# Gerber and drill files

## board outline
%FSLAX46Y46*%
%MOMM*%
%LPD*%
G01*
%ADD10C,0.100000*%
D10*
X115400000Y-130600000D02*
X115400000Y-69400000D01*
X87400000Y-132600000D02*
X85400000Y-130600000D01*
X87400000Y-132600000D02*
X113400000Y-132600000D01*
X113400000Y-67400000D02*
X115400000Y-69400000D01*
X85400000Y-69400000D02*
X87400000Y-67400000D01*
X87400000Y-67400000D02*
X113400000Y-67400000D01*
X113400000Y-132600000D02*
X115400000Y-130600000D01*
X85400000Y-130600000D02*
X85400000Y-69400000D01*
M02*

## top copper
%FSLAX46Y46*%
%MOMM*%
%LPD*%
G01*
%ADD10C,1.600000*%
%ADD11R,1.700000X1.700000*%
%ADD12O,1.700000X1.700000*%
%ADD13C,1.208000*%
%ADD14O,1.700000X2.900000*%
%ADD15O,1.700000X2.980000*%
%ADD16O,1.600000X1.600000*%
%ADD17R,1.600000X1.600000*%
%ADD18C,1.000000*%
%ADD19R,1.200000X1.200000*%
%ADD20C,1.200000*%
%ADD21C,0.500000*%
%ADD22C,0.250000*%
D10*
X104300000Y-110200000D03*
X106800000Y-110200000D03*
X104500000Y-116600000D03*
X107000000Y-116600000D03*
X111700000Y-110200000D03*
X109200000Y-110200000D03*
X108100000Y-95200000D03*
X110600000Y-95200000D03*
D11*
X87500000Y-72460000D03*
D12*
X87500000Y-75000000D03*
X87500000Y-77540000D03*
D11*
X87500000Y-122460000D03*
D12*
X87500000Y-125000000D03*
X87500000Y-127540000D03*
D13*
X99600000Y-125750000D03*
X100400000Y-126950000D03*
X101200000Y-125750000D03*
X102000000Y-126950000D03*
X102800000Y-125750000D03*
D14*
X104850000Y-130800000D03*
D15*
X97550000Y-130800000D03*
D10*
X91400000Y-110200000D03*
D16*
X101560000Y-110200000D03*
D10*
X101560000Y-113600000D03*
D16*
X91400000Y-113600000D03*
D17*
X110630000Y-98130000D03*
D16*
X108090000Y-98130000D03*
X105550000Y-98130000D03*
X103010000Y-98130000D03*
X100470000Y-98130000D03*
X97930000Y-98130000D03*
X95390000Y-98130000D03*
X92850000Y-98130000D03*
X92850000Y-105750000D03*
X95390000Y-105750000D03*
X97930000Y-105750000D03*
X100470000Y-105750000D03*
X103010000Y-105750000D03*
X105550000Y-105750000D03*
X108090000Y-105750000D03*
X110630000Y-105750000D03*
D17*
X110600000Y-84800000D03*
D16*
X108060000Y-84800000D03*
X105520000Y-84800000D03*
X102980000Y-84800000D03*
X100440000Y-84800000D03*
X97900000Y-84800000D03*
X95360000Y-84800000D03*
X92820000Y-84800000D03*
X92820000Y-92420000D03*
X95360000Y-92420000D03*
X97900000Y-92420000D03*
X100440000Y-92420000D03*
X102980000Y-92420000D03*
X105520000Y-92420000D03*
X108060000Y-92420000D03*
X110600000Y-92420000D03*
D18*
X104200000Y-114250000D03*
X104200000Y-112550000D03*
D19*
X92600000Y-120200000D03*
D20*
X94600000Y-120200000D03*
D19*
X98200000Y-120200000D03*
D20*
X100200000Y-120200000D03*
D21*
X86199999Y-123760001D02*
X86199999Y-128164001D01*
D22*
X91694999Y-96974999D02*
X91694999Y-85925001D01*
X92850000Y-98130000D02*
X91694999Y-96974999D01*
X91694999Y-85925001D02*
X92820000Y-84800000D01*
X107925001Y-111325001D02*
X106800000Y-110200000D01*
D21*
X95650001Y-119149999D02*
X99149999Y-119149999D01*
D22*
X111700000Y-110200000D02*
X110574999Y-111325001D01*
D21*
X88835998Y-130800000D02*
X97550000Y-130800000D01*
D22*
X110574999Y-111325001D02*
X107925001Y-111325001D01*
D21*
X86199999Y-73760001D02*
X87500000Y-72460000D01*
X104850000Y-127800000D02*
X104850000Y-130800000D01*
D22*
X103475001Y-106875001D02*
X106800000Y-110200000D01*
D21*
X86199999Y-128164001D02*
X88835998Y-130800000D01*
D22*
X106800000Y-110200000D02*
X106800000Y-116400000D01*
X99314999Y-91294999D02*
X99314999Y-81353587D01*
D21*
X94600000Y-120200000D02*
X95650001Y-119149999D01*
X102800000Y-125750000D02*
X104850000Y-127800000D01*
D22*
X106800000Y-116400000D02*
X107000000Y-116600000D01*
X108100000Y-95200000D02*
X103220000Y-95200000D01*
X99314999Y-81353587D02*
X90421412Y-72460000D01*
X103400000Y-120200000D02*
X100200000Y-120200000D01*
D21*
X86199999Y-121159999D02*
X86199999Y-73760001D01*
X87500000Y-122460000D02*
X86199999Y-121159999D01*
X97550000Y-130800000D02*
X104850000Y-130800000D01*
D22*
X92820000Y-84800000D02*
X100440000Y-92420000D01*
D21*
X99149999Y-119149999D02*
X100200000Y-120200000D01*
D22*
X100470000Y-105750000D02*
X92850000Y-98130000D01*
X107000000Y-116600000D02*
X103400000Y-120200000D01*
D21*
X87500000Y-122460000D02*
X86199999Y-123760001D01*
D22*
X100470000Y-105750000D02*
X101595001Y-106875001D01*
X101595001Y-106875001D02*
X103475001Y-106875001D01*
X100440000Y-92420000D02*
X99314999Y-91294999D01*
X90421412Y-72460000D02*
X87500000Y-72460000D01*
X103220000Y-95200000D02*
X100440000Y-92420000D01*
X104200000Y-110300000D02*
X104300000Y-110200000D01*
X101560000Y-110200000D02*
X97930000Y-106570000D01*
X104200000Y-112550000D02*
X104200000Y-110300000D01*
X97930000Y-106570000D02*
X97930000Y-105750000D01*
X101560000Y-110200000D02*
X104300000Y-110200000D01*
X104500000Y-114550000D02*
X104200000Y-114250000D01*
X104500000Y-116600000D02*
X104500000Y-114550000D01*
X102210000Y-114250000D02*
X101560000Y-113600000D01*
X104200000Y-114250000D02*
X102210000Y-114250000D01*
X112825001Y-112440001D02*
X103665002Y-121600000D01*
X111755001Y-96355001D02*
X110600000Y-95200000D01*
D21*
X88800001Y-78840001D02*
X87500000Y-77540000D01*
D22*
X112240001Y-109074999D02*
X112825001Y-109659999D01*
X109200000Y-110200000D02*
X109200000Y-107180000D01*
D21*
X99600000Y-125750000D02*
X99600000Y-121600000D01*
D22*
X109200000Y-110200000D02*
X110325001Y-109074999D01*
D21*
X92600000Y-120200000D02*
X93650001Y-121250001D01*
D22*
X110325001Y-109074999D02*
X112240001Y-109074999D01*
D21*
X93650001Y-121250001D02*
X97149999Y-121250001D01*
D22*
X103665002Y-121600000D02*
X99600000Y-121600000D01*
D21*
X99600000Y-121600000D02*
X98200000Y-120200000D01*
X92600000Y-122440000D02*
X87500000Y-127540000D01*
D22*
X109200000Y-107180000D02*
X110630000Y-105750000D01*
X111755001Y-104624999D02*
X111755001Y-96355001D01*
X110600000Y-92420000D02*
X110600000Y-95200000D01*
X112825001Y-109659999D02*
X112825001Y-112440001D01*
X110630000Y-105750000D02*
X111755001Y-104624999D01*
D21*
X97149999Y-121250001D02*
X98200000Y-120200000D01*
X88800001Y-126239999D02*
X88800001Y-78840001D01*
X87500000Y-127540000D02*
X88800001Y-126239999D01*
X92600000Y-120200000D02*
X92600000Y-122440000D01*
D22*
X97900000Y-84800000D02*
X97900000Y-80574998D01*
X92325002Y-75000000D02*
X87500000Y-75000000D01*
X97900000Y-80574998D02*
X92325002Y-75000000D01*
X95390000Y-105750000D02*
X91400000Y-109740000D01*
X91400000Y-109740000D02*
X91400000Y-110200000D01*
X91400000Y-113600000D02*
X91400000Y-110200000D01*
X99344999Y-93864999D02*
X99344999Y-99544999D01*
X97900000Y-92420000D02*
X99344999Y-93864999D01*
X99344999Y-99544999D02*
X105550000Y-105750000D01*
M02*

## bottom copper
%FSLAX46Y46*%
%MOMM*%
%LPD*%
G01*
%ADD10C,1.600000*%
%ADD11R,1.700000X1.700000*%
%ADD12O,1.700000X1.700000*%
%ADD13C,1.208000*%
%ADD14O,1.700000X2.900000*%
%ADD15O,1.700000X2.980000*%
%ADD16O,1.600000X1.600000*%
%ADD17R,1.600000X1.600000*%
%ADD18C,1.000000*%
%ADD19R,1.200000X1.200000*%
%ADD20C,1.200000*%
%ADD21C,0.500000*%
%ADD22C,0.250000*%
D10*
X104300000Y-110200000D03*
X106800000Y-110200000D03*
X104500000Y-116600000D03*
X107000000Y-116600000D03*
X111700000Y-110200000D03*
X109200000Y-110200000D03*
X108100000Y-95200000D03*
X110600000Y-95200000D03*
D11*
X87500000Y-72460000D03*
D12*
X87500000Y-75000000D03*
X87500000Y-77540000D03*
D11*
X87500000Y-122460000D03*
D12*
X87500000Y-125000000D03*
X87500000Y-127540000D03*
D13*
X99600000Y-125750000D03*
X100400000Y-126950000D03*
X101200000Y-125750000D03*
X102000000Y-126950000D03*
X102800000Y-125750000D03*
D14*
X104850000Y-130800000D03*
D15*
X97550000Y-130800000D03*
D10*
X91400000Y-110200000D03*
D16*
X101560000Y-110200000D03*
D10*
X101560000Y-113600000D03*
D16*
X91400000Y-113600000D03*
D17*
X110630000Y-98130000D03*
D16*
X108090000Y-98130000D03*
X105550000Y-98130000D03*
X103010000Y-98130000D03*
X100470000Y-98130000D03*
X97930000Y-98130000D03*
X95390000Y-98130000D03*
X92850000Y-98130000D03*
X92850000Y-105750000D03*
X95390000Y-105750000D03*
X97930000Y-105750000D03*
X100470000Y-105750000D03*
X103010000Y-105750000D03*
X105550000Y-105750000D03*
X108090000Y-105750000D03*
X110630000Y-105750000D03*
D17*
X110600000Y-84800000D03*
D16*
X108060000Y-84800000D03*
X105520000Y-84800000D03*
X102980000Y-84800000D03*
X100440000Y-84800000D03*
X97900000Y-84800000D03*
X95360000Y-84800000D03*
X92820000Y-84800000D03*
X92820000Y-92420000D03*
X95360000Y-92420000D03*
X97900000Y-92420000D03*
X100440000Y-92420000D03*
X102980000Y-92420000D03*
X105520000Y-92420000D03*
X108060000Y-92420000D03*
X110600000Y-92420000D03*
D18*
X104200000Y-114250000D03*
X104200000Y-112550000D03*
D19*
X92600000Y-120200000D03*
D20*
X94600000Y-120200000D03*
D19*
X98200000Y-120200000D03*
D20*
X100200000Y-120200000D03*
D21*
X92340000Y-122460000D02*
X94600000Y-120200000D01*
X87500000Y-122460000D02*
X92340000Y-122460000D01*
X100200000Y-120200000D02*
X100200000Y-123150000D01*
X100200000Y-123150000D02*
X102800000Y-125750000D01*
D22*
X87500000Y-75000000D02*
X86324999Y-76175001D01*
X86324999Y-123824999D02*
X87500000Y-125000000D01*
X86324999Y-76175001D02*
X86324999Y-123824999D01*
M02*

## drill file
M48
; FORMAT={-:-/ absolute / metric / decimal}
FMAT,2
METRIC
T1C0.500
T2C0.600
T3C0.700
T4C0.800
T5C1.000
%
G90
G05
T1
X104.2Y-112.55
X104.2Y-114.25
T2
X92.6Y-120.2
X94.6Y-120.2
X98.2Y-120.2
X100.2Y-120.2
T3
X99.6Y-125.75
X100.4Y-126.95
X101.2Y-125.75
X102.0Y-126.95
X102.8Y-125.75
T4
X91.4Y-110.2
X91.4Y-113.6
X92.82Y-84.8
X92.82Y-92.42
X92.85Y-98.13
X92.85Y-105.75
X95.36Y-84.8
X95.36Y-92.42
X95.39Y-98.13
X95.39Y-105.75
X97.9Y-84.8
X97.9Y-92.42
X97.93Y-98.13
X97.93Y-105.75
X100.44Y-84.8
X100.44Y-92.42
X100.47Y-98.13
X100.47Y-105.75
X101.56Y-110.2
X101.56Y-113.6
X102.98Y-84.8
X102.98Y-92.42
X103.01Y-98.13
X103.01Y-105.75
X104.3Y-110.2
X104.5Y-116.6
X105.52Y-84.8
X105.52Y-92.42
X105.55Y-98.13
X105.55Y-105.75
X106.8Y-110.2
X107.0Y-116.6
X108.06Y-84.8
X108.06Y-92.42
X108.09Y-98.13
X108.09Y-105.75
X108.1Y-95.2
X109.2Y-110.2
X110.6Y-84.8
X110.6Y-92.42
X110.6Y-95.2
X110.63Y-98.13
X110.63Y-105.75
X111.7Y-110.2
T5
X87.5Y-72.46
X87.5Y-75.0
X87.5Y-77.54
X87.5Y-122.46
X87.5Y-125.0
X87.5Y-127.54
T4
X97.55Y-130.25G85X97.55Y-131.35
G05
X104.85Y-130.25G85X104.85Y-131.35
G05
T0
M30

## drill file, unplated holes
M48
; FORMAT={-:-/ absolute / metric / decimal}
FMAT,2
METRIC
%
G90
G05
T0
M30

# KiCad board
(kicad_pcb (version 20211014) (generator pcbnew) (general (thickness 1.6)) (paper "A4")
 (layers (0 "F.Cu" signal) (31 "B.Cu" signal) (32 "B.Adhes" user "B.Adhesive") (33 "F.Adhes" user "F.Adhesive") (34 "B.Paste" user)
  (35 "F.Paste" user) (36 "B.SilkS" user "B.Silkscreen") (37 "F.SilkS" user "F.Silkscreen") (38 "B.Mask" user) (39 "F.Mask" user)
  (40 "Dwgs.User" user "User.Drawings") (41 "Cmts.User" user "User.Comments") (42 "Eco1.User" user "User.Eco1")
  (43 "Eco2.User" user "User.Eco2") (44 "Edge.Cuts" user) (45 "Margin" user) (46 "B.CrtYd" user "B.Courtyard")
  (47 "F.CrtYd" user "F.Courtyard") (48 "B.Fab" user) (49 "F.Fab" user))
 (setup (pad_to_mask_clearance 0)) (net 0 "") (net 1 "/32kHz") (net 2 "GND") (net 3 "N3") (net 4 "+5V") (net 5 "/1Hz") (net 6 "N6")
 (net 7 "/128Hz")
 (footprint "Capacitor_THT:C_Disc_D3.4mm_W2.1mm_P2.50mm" (layer "F.Cu") (at 104.3 110.2)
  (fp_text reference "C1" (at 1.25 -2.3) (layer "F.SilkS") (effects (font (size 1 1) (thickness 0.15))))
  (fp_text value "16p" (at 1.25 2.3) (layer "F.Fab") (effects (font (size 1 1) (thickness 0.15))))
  (pad "1" thru_hole circle locked (at 0 0) (size 1.6 1.6) (drill 0.8) (layers *.Cu *.Mask) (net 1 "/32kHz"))
  (pad "2" thru_hole circle locked (at 2.5 0) (size 1.6 1.6) (drill 0.8) (layers *.Cu *.Mask) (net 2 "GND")))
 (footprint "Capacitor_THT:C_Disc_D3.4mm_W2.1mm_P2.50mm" (layer "F.Cu") (at 104.5 116.6)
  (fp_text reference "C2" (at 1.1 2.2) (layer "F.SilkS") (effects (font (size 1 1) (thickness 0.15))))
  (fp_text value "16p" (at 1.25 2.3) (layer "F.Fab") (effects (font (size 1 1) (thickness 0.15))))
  (pad "1" thru_hole circle locked (at 0 0) (size 1.6 1.6) (drill 0.8) (layers *.Cu *.Mask) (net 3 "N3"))
  (pad "2" thru_hole circle locked (at 2.5 0) (size 1.6 1.6) (drill 0.8) (layers *.Cu *.Mask) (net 2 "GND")))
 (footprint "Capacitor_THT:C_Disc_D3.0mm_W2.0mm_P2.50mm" (layer "F.Cu") (at 111.7 110.2 180)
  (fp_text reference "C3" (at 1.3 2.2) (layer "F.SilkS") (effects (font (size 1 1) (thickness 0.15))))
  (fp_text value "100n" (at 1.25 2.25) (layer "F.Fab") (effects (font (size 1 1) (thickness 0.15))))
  (pad "1" thru_hole circle locked (at 0 0 180) (size 1.6 1.6) (drill 0.8) (layers *.Cu *.Mask) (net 2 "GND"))
  (pad "2" thru_hole circle locked (at 2.5 0 180) (size 1.6 1.6) (drill 0.8) (layers *.Cu *.Mask) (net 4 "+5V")))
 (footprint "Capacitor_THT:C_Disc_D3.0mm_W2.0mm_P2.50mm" (layer "F.Cu") (at 108.1 95.2)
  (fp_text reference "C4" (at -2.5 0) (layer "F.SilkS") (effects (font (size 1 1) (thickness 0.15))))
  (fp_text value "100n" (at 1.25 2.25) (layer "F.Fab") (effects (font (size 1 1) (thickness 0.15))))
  (pad "1" thru_hole circle locked (at 0 0) (size 1.6 1.6) (drill 0.8) (layers *.Cu *.Mask) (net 2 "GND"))
  (pad "2" thru_hole circle locked (at 2.5 0) (size 1.6 1.6) (drill 0.8) (layers *.Cu *.Mask) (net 4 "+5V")))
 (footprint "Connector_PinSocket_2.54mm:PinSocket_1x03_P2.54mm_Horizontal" (layer "F.Cu") (at 87.5 72.46)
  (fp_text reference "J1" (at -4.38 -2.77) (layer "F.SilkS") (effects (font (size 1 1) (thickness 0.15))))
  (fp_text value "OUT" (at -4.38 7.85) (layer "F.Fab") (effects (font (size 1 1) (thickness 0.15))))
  (pad "1" thru_hole rect locked (at 0 0) (size 1.7 1.7) (drill 1) (layers *.Cu *.Mask) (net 2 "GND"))
  (pad "2" thru_hole oval locked (at 0 2.54) (size 1.7 1.7) (drill 1) (layers *.Cu *.Mask) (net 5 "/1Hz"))
  (pad "3" thru_hole oval locked (at 0 5.08) (size 1.7 1.7) (drill 1) (layers *.Cu *.Mask) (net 4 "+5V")))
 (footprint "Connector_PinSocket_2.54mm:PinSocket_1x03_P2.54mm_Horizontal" (layer "F.Cu") (at 87.5 122.46)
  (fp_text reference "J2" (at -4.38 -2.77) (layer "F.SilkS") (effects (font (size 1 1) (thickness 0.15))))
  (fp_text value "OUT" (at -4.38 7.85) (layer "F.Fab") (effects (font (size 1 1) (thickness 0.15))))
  (pad "1" thru_hole rect locked (at 0 0) (size 1.7 1.7) (drill 1) (layers *.Cu *.Mask) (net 2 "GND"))
  (pad "2" thru_hole oval locked (at 0 2.54) (size 1.7 1.7) (drill 1) (layers *.Cu *.Mask) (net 5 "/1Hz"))
  (pad "3" thru_hole oval locked (at 0 5.08) (size 1.7 1.7) (drill 1) (layers *.Cu *.Mask) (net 4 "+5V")))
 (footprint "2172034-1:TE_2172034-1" (layer "F.Cu") (at 101.2 130.8 -90)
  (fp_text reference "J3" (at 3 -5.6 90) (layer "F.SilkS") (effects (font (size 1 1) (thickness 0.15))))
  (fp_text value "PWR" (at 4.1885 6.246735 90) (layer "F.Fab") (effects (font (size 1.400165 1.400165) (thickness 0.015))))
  (pad "1" thru_hole circle locked (at -5.05 1.6 270) (size 1.208 1.208) (drill 0.7) (layers *.Cu *.Mask) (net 4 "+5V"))
  (pad "2" thru_hole circle locked (at -3.85 0.8 270) (size 1.208 1.208) (drill 0.7) (layers *.Cu *.Mask))
  (pad "3" thru_hole circle locked (at -5.05 0 270) (size 1.208 1.208) (drill 0.7) (layers *.Cu *.Mask))
  (pad "4" thru_hole circle locked (at -3.85 -0.8 270) (size 1.208 1.208) (drill 0.7) (layers *.Cu *.Mask))
  (pad "5" thru_hole circle locked (at -5.05 -1.6 270) (size 1.208 1.208) (drill 0.7) (layers *.Cu *.Mask) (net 2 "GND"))
  (pad "6" thru_hole oval locked (at 0 -3.65 270) (size 2.9 1.7) (drill oval 1.9 0.8) (layers *.Cu *.Mask) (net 2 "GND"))
  (pad "6" thru_hole oval locked (at 0 3.65 270) (size 2.98 1.7) (drill oval 1.9 0.8) (layers *.Cu *.Mask) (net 2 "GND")))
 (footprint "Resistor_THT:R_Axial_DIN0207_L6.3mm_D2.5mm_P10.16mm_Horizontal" (layer "F.Cu") (at 91.4 110.2)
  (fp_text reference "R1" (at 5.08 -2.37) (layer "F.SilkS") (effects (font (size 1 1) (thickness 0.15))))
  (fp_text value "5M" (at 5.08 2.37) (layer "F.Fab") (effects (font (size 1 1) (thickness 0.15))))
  (pad "1" thru_hole circle locked (at 0 0) (size 1.6 1.6) (drill 0.8) (layers *.Cu *.Mask) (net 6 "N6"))
  (pad "2" thru_hole oval locked (at 10.16 0) (size 1.6 1.6) (drill 0.8) (layers *.Cu *.Mask) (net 1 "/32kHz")))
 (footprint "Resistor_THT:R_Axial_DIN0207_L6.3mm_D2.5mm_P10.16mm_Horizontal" (layer "F.Cu") (at 101.56 113.6 180)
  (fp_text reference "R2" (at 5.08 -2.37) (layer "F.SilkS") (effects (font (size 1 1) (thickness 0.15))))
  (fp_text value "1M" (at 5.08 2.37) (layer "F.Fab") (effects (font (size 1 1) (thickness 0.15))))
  (pad "1" thru_hole circle locked (at 0 0 180) (size 1.6 1.6) (drill 0.8) (layers *.Cu *.Mask) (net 3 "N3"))
  (pad "2" thru_hole oval locked (at 10.16 0 180) (size 1.6 1.6) (drill 0.8) (layers *.Cu *.Mask) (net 6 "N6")))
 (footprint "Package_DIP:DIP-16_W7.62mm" (layer "F.Cu") (at 110.63 98.13 -90)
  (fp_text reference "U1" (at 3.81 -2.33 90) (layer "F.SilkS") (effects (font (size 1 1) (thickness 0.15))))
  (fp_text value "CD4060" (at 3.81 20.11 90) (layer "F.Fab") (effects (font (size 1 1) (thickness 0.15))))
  (pad "1" thru_hole rect locked (at 0 0 270) (size 1.6 1.6) (drill 0.8) (layers *.Cu *.Mask))
  (pad "2" thru_hole oval locked (at 0 2.54 270) (size 1.6 1.6) (drill 0.8) (layers *.Cu *.Mask))
  (pad "3" thru_hole oval locked (at 0 5.08 270) (size 1.6 1.6) (drill 0.8) (layers *.Cu *.Mask))
  (pad "4" thru_hole oval locked (at 0 7.62 270) (size 1.6 1.6) (drill 0.8) (layers *.Cu *.Mask))
  (pad "5" thru_hole oval locked (at 0 10.16 270) (size 1.6 1.6) (drill 0.8) (layers *.Cu *.Mask))
  (pad "6" thru_hole oval locked (at 0 12.7 270) (size 1.6 1.6) (drill 0.8) (layers *.Cu *.Mask))
  (pad "7" thru_hole oval locked (at 0 15.24 270) (size 1.6 1.6) (drill 0.8) (layers *.Cu *.Mask))
  (pad "8" thru_hole oval locked (at 0 17.78 270) (size 1.6 1.6) (drill 0.8) (layers *.Cu *.Mask) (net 2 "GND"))
  (pad "9" thru_hole oval locked (at 7.62 17.78 270) (size 1.6 1.6) (drill 0.8) (layers *.Cu *.Mask))
  (pad "10" thru_hole oval locked (at 7.62 15.24 270) (size 1.6 1.6) (drill 0.8) (layers *.Cu *.Mask) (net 6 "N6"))
  (pad "11" thru_hole oval locked (at 7.62 12.7 270) (size 1.6 1.6) (drill 0.8) (layers *.Cu *.Mask) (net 1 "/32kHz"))
  (pad "12" thru_hole oval locked (at 7.62 10.16 270) (size 1.6 1.6) (drill 0.8) (layers *.Cu *.Mask) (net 2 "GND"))
  (pad "13" thru_hole oval locked (at 7.62 7.62 270) (size 1.6 1.6) (drill 0.8) (layers *.Cu *.Mask))
  (pad "14" thru_hole oval locked (at 7.62 5.08 270) (size 1.6 1.6) (drill 0.8) (layers *.Cu *.Mask) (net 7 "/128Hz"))
  (pad "15" thru_hole oval locked (at 7.62 2.54 270) (size 1.6 1.6) (drill 0.8) (layers *.Cu *.Mask))
  (pad "16" thru_hole oval locked (at 7.62 0 270) (size 1.6 1.6) (drill 0.8) (layers *.Cu *.Mask) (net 4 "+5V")))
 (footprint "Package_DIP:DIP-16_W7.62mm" (layer "F.Cu") (at 110.6 84.8 -90)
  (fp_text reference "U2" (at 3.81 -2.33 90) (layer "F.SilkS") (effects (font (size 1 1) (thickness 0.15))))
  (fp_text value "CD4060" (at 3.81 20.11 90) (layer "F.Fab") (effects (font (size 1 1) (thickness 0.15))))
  (pad "1" thru_hole rect locked (at 0 0 270) (size 1.6 1.6) (drill 0.8) (layers *.Cu *.Mask))
  (pad "2" thru_hole oval locked (at 0 2.54 270) (size 1.6 1.6) (drill 0.8) (layers *.Cu *.Mask))
  (pad "3" thru_hole oval locked (at 0 5.08 270) (size 1.6 1.6) (drill 0.8) (layers *.Cu *.Mask))
  (pad "4" thru_hole oval locked (at 0 7.62 270) (size 1.6 1.6) (drill 0.8) (layers *.Cu *.Mask))
  (pad "5" thru_hole oval locked (at 0 10.16 270) (size 1.6 1.6) (drill 0.8) (layers *.Cu *.Mask))
  (pad "6" thru_hole oval locked (at 0 12.7 270) (size 1.6 1.6) (drill 0.8) (layers *.Cu *.Mask) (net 5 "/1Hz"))
  (pad "7" thru_hole oval locked (at 0 15.24 270) (size 1.6 1.6) (drill 0.8) (layers *.Cu *.Mask))
  (pad "8" thru_hole oval locked (at 0 17.78 270) (size 1.6 1.6) (drill 0.8) (layers *.Cu *.Mask) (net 2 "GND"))
  (pad "9" thru_hole oval locked (at 7.62 17.78 270) (size 1.6 1.6) (drill 0.8) (layers *.Cu *.Mask))
  (pad "10" thru_hole oval locked (at 7.62 15.24 270) (size 1.6 1.6) (drill 0.8) (layers *.Cu *.Mask))
  (pad "11" thru_hole oval locked (at 7.62 12.7 270) (size 1.6 1.6) (drill 0.8) (layers *.Cu *.Mask) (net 7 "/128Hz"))
  (pad "12" thru_hole oval locked (at 7.62 10.16 270) (size 1.6 1.6) (drill 0.8) (layers *.Cu *.Mask) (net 2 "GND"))
  (pad "13" thru_hole oval locked (at 7.62 7.62 270) (size 1.6 1.6) (drill 0.8) (layers *.Cu *.Mask))
  (pad "14" thru_hole oval locked (at 7.62 5.08 270) (size 1.6 1.6) (drill 0.8) (layers *.Cu *.Mask))
  (pad "15" thru_hole oval locked (at 7.62 2.54 270) (size 1.6 1.6) (drill 0.8) (layers *.Cu *.Mask))
  (pad "16" thru_hole oval locked (at 7.62 0 270) (size 1.6 1.6) (drill 0.8) (layers *.Cu *.Mask) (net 4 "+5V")))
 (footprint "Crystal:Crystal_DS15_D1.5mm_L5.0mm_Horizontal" (layer "F.Cu") (at 104.2 114.25 90)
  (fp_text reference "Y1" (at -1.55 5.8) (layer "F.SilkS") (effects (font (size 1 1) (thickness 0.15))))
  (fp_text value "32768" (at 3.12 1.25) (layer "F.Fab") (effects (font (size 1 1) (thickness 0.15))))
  (pad "1" thru_hole circle locked (at 0 0 90) (size 1 1) (drill 0.5) (layers *.Cu *.Mask) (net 3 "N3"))
  (pad "2" thru_hole circle locked (at 1.7 0 90) (size 1 1) (drill 0.5) (layers *.Cu *.Mask) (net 1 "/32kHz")))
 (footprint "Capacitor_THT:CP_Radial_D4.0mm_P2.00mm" (layer "F.Cu") (at 92.6 120.2)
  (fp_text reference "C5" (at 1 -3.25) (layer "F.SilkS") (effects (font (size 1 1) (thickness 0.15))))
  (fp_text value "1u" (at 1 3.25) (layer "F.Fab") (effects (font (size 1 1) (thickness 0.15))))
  (pad "1" thru_hole rect locked (at 0 0) (size 1.2 1.2) (drill 0.6) (layers *.Cu *.Mask) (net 4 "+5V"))
  (pad "2" thru_hole circle locked (at 2 0) (size 1.2 1.2) (drill 0.6) (layers *.Cu *.Mask) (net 2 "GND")))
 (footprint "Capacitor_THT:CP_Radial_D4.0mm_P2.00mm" (layer "F.Cu") (at 98.2 120.2)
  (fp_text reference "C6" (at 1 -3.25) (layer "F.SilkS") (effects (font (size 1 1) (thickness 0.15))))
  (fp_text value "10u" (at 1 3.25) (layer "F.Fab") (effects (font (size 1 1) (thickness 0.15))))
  (pad "1" thru_hole rect locked (at 0 0) (size 1.2 1.2) (drill 0.6) (layers *.Cu *.Mask) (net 4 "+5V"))
  (pad "2" thru_hole circle locked (at 2 0) (size 1.2 1.2) (drill 0.6) (layers *.Cu *.Mask) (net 2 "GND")))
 (gr_line (start 115.4 130.6) (end 115.4 69.4) (layer "Edge.Cuts") (width 0.1))
 (gr_line (start 87.4 132.6) (end 85.4 130.6) (layer "Edge.Cuts") (width 0.1))
 (gr_line (start 87.4 132.6) (end 113.4 132.6) (layer "Edge.Cuts") (width 0.1))
 (gr_line (start 113.4 67.4) (end 115.4 69.4) (layer "Edge.Cuts") (width 0.1))
 (gr_line (start 85.4 69.4) (end 87.4 67.4) (layer "Edge.Cuts") (width 0.1))
 (gr_line (start 87.4 67.4) (end 113.4 67.4) (layer "Edge.Cuts") (width 0.1))
 (gr_line (start 113.4 132.6) (end 115.4 130.6) (layer "Edge.Cuts") (width 0.1))
 (gr_line (start 85.4 130.6) (end 85.4 69.4) (layer "Edge.Cuts") (width 0.1))
 (segment (start 86.199999 123.760001) (end 86.199999 128.164001) (width 0.5) (layer "F.Cu") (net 2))
 (segment (start 91.694999 96.974999) (end 91.694999 85.925001) (width 0.25) (layer "F.Cu") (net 2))
 (segment (start 92.85 98.13) (end 91.694999 96.974999) (width 0.25) (layer "F.Cu") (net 2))
 (segment (start 91.694999 85.925001) (end 92.82 84.8) (width 0.25) (layer "F.Cu") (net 2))
 (segment (start 107.925001 111.325001) (end 106.8 110.2) (width 0.25) (layer "F.Cu") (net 2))
 (segment (start 95.650001 119.149999) (end 99.149999 119.149999) (width 0.5) (layer "F.Cu") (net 2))
 (segment (start 111.7 110.2) (end 110.574999 111.325001) (width 0.25) (layer "F.Cu") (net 2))
 (segment (start 88.835998 130.8) (end 97.55 130.8) (width 0.5) (layer "F.Cu") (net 2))
 (segment (start 110.574999 111.325001) (end 107.925001 111.325001) (width 0.25) (layer "F.Cu") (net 2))
 (segment (start 86.199999 73.760001) (end 87.5 72.46) (width 0.5) (layer "F.Cu") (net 2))
 (segment (start 104.85 127.8) (end 104.85 130.8) (width 0.5) (layer "F.Cu") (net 2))
 (segment (start 103.475001 106.875001) (end 106.8 110.2) (width 0.25) (layer "F.Cu") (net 2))
 (segment (start 86.199999 128.164001) (end 88.835998 130.8) (width 0.5) (layer "F.Cu") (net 2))
 (segment (start 106.8 110.2) (end 106.8 116.4) (width 0.25) (layer "F.Cu") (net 2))
 (segment (start 99.314999 91.294999) (end 99.314999 81.353587) (width 0.25) (layer "F.Cu") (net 2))
 (segment (start 94.6 120.2) (end 95.650001 119.149999) (width 0.5) (layer "F.Cu") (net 2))
 (segment (start 102.8 125.75) (end 104.85 127.8) (width 0.5) (layer "F.Cu") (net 2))
 (segment (start 106.8 116.4) (end 107 116.6) (width 0.25) (layer "F.Cu") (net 2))
 (segment (start 108.1 95.2) (end 103.22 95.2) (width 0.25) (layer "F.Cu") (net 2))
 (segment (start 99.314999 81.353587) (end 90.421412 72.46) (width 0.25) (layer "F.Cu") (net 2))
 (segment (start 103.4 120.2) (end 100.2 120.2) (width 0.25) (layer "F.Cu") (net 2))
 (segment (start 86.199999 121.159999) (end 86.199999 73.760001) (width 0.5) (layer "F.Cu") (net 2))
 (segment (start 87.5 122.46) (end 86.199999 121.159999) (width 0.5) (layer "F.Cu") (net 2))
 (segment (start 97.55 130.8) (end 104.85 130.8) (width 0.5) (layer "F.Cu") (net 2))
 (segment (start 92.82 84.8) (end 100.44 92.42) (width 0.25) (layer "F.Cu") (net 2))
 (segment (start 99.149999 119.149999) (end 100.2 120.2) (width 0.5) (layer "F.Cu") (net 2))
 (segment (start 100.47 105.75) (end 92.85 98.13) (width 0.25) (layer "F.Cu") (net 2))
 (segment (start 107 116.6) (end 103.4 120.2) (width 0.25) (layer "F.Cu") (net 2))
 (segment (start 87.5 122.46) (end 86.199999 123.760001) (width 0.5) (layer "F.Cu") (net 2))
 (segment (start 100.47 105.75) (end 101.595001 106.875001) (width 0.25) (layer "F.Cu") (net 2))
 (segment (start 101.595001 106.875001) (end 103.475001 106.875001) (width 0.25) (layer "F.Cu") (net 2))
 (segment (start 100.44 92.42) (end 99.314999 91.294999) (width 0.25) (layer "F.Cu") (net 2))
 (segment (start 90.421412 72.46) (end 87.5 72.46) (width 0.25) (layer "F.Cu") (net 2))
 (segment (start 103.22 95.2) (end 100.44 92.42) (width 0.25) (layer "F.Cu") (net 2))
 (segment (start 92.34 122.46) (end 94.6 120.2) (width 0.5) (layer "B.Cu") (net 2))
 (segment (start 87.5 122.46) (end 92.34 122.46) (width 0.5) (layer "B.Cu") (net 2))
 (segment (start 100.2 120.2) (end 100.2 123.15) (width 0.5) (layer "B.Cu") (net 2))
 (segment (start 100.2 123.15) (end 102.8 125.75) (width 0.5) (layer "B.Cu") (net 2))
 (segment (start 104.2 110.3) (end 104.3 110.2) (width 0.25) (layer "F.Cu") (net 1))
 (segment (start 101.56 110.2) (end 97.93 106.57) (width 0.25) (layer "F.Cu") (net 1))
 (segment (start 104.2 112.55) (end 104.2 110.3) (width 0.25) (layer "F.Cu") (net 1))
 (segment (start 97.93 106.57) (end 97.93 105.75) (width 0.25) (layer "F.Cu") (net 1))
 (segment (start 101.56 110.2) (end 104.3 110.2) (width 0.25) (layer "F.Cu") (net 1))
 (segment (start 104.5 114.55) (end 104.2 114.25) (width 0.25) (layer "F.Cu") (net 3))
 (segment (start 104.5 116.6) (end 104.5 114.55) (width 0.25) (layer "F.Cu") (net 3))
 (segment (start 102.21 114.25) (end 101.56 113.6) (width 0.25) (layer "F.Cu") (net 3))
 (segment (start 104.2 114.25) (end 102.21 114.25) (width 0.25) (layer "F.Cu") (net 3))
 (segment (start 112.825001 112.440001) (end 103.665002 121.6) (width 0.25) (layer "F.Cu") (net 4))
 (segment (start 111.755001 96.355001) (end 110.6 95.2) (width 0.25) (layer "F.Cu") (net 4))
 (segment (start 88.800001 78.840001) (end 87.5 77.54) (width 0.5) (layer "F.Cu") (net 4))
 (segment (start 112.240001 109.074999) (end 112.825001 109.659999) (width 0.25) (layer "F.Cu") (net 4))
 (segment (start 109.2 110.2) (end 109.2 107.18) (width 0.25) (layer "F.Cu") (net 4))
 (segment (start 99.6 125.75) (end 99.6 121.6) (width 0.5) (layer "F.Cu") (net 4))
 (segment (start 109.2 110.2) (end 110.325001 109.074999) (width 0.25) (layer "F.Cu") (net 4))
 (segment (start 92.6 120.2) (end 93.650001 121.250001) (width 0.5) (layer "F.Cu") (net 4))
 (segment (start 110.325001 109.074999) (end 112.240001 109.074999) (width 0.25) (layer "F.Cu") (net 4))
 (segment (start 93.650001 121.250001) (end 97.149999 121.250001) (width 0.5) (layer "F.Cu") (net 4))
 (segment (start 103.665002 121.6) (end 99.6 121.6) (width 0.25) (layer "F.Cu") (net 4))
 (segment (start 99.6 121.6) (end 98.2 120.2) (width 0.5) (layer "F.Cu") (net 4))
 (segment (start 92.6 122.44) (end 87.5 127.54) (width 0.5) (layer "F.Cu") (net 4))
 (segment (start 109.2 107.18) (end 110.63 105.75) (width 0.25) (layer "F.Cu") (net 4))
 (segment (start 111.755001 104.624999) (end 111.755001 96.355001) (width 0.25) (layer "F.Cu") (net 4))
 (segment (start 110.6 92.42) (end 110.6 95.2) (width 0.25) (layer "F.Cu") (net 4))
 (segment (start 112.825001 109.659999) (end 112.825001 112.440001) (width 0.25) (layer "F.Cu") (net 4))
 (segment (start 110.63 105.75) (end 111.755001 104.624999) (width 0.25) (layer "F.Cu") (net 4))
 (segment (start 97.149999 121.250001) (end 98.2 120.2) (width 0.5) (layer "F.Cu") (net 4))
 (segment (start 88.800001 126.239999) (end 88.800001 78.840001) (width 0.5) (layer "F.Cu") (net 4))
 (segment (start 87.5 127.54) (end 88.800001 126.239999) (width 0.5) (layer "F.Cu") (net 4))
 (segment (start 92.6 120.2) (end 92.6 122.44) (width 0.5) (layer "F.Cu") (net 4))
 (segment (start 97.9 84.8) (end 97.9 80.574998) (width 0.25) (layer "F.Cu") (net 5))
 (segment (start 92.325002 75) (end 87.5 75) (width 0.25) (layer "F.Cu") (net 5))
 (segment (start 97.9 80.574998) (end 92.325002 75) (width 0.25) (layer "F.Cu") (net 5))
 (segment (start 87.5 75) (end 86.324999 76.175001) (width 0.25) (layer "B.Cu") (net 5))
 (segment (start 86.324999 123.824999) (end 87.5 125) (width 0.25) (layer "B.Cu") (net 5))
 (segment (start 86.324999 76.175001) (end 86.324999 123.824999) (width 0.25) (layer "B.Cu") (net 5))
 (segment (start 95.39 105.75) (end 91.4 109.74) (width 0.25) (layer "F.Cu") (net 6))
 (segment (start 91.4 109.74) (end 91.4 110.2) (width 0.25) (layer "F.Cu") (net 6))
 (segment (start 91.4 113.6) (end 91.4 110.2) (width 0.25) (layer "F.Cu") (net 6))
 (segment (start 99.344999 93.864999) (end 99.344999 99.544999) (width 0.25) (layer "F.Cu") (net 7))
 (segment (start 97.9 92.42) (end 99.344999 93.864999) (width 0.25) (layer "F.Cu") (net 7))
 (segment (start 99.344999 99.544999) (end 105.55 105.75) (width 0.25) (layer "F.Cu") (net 7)))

